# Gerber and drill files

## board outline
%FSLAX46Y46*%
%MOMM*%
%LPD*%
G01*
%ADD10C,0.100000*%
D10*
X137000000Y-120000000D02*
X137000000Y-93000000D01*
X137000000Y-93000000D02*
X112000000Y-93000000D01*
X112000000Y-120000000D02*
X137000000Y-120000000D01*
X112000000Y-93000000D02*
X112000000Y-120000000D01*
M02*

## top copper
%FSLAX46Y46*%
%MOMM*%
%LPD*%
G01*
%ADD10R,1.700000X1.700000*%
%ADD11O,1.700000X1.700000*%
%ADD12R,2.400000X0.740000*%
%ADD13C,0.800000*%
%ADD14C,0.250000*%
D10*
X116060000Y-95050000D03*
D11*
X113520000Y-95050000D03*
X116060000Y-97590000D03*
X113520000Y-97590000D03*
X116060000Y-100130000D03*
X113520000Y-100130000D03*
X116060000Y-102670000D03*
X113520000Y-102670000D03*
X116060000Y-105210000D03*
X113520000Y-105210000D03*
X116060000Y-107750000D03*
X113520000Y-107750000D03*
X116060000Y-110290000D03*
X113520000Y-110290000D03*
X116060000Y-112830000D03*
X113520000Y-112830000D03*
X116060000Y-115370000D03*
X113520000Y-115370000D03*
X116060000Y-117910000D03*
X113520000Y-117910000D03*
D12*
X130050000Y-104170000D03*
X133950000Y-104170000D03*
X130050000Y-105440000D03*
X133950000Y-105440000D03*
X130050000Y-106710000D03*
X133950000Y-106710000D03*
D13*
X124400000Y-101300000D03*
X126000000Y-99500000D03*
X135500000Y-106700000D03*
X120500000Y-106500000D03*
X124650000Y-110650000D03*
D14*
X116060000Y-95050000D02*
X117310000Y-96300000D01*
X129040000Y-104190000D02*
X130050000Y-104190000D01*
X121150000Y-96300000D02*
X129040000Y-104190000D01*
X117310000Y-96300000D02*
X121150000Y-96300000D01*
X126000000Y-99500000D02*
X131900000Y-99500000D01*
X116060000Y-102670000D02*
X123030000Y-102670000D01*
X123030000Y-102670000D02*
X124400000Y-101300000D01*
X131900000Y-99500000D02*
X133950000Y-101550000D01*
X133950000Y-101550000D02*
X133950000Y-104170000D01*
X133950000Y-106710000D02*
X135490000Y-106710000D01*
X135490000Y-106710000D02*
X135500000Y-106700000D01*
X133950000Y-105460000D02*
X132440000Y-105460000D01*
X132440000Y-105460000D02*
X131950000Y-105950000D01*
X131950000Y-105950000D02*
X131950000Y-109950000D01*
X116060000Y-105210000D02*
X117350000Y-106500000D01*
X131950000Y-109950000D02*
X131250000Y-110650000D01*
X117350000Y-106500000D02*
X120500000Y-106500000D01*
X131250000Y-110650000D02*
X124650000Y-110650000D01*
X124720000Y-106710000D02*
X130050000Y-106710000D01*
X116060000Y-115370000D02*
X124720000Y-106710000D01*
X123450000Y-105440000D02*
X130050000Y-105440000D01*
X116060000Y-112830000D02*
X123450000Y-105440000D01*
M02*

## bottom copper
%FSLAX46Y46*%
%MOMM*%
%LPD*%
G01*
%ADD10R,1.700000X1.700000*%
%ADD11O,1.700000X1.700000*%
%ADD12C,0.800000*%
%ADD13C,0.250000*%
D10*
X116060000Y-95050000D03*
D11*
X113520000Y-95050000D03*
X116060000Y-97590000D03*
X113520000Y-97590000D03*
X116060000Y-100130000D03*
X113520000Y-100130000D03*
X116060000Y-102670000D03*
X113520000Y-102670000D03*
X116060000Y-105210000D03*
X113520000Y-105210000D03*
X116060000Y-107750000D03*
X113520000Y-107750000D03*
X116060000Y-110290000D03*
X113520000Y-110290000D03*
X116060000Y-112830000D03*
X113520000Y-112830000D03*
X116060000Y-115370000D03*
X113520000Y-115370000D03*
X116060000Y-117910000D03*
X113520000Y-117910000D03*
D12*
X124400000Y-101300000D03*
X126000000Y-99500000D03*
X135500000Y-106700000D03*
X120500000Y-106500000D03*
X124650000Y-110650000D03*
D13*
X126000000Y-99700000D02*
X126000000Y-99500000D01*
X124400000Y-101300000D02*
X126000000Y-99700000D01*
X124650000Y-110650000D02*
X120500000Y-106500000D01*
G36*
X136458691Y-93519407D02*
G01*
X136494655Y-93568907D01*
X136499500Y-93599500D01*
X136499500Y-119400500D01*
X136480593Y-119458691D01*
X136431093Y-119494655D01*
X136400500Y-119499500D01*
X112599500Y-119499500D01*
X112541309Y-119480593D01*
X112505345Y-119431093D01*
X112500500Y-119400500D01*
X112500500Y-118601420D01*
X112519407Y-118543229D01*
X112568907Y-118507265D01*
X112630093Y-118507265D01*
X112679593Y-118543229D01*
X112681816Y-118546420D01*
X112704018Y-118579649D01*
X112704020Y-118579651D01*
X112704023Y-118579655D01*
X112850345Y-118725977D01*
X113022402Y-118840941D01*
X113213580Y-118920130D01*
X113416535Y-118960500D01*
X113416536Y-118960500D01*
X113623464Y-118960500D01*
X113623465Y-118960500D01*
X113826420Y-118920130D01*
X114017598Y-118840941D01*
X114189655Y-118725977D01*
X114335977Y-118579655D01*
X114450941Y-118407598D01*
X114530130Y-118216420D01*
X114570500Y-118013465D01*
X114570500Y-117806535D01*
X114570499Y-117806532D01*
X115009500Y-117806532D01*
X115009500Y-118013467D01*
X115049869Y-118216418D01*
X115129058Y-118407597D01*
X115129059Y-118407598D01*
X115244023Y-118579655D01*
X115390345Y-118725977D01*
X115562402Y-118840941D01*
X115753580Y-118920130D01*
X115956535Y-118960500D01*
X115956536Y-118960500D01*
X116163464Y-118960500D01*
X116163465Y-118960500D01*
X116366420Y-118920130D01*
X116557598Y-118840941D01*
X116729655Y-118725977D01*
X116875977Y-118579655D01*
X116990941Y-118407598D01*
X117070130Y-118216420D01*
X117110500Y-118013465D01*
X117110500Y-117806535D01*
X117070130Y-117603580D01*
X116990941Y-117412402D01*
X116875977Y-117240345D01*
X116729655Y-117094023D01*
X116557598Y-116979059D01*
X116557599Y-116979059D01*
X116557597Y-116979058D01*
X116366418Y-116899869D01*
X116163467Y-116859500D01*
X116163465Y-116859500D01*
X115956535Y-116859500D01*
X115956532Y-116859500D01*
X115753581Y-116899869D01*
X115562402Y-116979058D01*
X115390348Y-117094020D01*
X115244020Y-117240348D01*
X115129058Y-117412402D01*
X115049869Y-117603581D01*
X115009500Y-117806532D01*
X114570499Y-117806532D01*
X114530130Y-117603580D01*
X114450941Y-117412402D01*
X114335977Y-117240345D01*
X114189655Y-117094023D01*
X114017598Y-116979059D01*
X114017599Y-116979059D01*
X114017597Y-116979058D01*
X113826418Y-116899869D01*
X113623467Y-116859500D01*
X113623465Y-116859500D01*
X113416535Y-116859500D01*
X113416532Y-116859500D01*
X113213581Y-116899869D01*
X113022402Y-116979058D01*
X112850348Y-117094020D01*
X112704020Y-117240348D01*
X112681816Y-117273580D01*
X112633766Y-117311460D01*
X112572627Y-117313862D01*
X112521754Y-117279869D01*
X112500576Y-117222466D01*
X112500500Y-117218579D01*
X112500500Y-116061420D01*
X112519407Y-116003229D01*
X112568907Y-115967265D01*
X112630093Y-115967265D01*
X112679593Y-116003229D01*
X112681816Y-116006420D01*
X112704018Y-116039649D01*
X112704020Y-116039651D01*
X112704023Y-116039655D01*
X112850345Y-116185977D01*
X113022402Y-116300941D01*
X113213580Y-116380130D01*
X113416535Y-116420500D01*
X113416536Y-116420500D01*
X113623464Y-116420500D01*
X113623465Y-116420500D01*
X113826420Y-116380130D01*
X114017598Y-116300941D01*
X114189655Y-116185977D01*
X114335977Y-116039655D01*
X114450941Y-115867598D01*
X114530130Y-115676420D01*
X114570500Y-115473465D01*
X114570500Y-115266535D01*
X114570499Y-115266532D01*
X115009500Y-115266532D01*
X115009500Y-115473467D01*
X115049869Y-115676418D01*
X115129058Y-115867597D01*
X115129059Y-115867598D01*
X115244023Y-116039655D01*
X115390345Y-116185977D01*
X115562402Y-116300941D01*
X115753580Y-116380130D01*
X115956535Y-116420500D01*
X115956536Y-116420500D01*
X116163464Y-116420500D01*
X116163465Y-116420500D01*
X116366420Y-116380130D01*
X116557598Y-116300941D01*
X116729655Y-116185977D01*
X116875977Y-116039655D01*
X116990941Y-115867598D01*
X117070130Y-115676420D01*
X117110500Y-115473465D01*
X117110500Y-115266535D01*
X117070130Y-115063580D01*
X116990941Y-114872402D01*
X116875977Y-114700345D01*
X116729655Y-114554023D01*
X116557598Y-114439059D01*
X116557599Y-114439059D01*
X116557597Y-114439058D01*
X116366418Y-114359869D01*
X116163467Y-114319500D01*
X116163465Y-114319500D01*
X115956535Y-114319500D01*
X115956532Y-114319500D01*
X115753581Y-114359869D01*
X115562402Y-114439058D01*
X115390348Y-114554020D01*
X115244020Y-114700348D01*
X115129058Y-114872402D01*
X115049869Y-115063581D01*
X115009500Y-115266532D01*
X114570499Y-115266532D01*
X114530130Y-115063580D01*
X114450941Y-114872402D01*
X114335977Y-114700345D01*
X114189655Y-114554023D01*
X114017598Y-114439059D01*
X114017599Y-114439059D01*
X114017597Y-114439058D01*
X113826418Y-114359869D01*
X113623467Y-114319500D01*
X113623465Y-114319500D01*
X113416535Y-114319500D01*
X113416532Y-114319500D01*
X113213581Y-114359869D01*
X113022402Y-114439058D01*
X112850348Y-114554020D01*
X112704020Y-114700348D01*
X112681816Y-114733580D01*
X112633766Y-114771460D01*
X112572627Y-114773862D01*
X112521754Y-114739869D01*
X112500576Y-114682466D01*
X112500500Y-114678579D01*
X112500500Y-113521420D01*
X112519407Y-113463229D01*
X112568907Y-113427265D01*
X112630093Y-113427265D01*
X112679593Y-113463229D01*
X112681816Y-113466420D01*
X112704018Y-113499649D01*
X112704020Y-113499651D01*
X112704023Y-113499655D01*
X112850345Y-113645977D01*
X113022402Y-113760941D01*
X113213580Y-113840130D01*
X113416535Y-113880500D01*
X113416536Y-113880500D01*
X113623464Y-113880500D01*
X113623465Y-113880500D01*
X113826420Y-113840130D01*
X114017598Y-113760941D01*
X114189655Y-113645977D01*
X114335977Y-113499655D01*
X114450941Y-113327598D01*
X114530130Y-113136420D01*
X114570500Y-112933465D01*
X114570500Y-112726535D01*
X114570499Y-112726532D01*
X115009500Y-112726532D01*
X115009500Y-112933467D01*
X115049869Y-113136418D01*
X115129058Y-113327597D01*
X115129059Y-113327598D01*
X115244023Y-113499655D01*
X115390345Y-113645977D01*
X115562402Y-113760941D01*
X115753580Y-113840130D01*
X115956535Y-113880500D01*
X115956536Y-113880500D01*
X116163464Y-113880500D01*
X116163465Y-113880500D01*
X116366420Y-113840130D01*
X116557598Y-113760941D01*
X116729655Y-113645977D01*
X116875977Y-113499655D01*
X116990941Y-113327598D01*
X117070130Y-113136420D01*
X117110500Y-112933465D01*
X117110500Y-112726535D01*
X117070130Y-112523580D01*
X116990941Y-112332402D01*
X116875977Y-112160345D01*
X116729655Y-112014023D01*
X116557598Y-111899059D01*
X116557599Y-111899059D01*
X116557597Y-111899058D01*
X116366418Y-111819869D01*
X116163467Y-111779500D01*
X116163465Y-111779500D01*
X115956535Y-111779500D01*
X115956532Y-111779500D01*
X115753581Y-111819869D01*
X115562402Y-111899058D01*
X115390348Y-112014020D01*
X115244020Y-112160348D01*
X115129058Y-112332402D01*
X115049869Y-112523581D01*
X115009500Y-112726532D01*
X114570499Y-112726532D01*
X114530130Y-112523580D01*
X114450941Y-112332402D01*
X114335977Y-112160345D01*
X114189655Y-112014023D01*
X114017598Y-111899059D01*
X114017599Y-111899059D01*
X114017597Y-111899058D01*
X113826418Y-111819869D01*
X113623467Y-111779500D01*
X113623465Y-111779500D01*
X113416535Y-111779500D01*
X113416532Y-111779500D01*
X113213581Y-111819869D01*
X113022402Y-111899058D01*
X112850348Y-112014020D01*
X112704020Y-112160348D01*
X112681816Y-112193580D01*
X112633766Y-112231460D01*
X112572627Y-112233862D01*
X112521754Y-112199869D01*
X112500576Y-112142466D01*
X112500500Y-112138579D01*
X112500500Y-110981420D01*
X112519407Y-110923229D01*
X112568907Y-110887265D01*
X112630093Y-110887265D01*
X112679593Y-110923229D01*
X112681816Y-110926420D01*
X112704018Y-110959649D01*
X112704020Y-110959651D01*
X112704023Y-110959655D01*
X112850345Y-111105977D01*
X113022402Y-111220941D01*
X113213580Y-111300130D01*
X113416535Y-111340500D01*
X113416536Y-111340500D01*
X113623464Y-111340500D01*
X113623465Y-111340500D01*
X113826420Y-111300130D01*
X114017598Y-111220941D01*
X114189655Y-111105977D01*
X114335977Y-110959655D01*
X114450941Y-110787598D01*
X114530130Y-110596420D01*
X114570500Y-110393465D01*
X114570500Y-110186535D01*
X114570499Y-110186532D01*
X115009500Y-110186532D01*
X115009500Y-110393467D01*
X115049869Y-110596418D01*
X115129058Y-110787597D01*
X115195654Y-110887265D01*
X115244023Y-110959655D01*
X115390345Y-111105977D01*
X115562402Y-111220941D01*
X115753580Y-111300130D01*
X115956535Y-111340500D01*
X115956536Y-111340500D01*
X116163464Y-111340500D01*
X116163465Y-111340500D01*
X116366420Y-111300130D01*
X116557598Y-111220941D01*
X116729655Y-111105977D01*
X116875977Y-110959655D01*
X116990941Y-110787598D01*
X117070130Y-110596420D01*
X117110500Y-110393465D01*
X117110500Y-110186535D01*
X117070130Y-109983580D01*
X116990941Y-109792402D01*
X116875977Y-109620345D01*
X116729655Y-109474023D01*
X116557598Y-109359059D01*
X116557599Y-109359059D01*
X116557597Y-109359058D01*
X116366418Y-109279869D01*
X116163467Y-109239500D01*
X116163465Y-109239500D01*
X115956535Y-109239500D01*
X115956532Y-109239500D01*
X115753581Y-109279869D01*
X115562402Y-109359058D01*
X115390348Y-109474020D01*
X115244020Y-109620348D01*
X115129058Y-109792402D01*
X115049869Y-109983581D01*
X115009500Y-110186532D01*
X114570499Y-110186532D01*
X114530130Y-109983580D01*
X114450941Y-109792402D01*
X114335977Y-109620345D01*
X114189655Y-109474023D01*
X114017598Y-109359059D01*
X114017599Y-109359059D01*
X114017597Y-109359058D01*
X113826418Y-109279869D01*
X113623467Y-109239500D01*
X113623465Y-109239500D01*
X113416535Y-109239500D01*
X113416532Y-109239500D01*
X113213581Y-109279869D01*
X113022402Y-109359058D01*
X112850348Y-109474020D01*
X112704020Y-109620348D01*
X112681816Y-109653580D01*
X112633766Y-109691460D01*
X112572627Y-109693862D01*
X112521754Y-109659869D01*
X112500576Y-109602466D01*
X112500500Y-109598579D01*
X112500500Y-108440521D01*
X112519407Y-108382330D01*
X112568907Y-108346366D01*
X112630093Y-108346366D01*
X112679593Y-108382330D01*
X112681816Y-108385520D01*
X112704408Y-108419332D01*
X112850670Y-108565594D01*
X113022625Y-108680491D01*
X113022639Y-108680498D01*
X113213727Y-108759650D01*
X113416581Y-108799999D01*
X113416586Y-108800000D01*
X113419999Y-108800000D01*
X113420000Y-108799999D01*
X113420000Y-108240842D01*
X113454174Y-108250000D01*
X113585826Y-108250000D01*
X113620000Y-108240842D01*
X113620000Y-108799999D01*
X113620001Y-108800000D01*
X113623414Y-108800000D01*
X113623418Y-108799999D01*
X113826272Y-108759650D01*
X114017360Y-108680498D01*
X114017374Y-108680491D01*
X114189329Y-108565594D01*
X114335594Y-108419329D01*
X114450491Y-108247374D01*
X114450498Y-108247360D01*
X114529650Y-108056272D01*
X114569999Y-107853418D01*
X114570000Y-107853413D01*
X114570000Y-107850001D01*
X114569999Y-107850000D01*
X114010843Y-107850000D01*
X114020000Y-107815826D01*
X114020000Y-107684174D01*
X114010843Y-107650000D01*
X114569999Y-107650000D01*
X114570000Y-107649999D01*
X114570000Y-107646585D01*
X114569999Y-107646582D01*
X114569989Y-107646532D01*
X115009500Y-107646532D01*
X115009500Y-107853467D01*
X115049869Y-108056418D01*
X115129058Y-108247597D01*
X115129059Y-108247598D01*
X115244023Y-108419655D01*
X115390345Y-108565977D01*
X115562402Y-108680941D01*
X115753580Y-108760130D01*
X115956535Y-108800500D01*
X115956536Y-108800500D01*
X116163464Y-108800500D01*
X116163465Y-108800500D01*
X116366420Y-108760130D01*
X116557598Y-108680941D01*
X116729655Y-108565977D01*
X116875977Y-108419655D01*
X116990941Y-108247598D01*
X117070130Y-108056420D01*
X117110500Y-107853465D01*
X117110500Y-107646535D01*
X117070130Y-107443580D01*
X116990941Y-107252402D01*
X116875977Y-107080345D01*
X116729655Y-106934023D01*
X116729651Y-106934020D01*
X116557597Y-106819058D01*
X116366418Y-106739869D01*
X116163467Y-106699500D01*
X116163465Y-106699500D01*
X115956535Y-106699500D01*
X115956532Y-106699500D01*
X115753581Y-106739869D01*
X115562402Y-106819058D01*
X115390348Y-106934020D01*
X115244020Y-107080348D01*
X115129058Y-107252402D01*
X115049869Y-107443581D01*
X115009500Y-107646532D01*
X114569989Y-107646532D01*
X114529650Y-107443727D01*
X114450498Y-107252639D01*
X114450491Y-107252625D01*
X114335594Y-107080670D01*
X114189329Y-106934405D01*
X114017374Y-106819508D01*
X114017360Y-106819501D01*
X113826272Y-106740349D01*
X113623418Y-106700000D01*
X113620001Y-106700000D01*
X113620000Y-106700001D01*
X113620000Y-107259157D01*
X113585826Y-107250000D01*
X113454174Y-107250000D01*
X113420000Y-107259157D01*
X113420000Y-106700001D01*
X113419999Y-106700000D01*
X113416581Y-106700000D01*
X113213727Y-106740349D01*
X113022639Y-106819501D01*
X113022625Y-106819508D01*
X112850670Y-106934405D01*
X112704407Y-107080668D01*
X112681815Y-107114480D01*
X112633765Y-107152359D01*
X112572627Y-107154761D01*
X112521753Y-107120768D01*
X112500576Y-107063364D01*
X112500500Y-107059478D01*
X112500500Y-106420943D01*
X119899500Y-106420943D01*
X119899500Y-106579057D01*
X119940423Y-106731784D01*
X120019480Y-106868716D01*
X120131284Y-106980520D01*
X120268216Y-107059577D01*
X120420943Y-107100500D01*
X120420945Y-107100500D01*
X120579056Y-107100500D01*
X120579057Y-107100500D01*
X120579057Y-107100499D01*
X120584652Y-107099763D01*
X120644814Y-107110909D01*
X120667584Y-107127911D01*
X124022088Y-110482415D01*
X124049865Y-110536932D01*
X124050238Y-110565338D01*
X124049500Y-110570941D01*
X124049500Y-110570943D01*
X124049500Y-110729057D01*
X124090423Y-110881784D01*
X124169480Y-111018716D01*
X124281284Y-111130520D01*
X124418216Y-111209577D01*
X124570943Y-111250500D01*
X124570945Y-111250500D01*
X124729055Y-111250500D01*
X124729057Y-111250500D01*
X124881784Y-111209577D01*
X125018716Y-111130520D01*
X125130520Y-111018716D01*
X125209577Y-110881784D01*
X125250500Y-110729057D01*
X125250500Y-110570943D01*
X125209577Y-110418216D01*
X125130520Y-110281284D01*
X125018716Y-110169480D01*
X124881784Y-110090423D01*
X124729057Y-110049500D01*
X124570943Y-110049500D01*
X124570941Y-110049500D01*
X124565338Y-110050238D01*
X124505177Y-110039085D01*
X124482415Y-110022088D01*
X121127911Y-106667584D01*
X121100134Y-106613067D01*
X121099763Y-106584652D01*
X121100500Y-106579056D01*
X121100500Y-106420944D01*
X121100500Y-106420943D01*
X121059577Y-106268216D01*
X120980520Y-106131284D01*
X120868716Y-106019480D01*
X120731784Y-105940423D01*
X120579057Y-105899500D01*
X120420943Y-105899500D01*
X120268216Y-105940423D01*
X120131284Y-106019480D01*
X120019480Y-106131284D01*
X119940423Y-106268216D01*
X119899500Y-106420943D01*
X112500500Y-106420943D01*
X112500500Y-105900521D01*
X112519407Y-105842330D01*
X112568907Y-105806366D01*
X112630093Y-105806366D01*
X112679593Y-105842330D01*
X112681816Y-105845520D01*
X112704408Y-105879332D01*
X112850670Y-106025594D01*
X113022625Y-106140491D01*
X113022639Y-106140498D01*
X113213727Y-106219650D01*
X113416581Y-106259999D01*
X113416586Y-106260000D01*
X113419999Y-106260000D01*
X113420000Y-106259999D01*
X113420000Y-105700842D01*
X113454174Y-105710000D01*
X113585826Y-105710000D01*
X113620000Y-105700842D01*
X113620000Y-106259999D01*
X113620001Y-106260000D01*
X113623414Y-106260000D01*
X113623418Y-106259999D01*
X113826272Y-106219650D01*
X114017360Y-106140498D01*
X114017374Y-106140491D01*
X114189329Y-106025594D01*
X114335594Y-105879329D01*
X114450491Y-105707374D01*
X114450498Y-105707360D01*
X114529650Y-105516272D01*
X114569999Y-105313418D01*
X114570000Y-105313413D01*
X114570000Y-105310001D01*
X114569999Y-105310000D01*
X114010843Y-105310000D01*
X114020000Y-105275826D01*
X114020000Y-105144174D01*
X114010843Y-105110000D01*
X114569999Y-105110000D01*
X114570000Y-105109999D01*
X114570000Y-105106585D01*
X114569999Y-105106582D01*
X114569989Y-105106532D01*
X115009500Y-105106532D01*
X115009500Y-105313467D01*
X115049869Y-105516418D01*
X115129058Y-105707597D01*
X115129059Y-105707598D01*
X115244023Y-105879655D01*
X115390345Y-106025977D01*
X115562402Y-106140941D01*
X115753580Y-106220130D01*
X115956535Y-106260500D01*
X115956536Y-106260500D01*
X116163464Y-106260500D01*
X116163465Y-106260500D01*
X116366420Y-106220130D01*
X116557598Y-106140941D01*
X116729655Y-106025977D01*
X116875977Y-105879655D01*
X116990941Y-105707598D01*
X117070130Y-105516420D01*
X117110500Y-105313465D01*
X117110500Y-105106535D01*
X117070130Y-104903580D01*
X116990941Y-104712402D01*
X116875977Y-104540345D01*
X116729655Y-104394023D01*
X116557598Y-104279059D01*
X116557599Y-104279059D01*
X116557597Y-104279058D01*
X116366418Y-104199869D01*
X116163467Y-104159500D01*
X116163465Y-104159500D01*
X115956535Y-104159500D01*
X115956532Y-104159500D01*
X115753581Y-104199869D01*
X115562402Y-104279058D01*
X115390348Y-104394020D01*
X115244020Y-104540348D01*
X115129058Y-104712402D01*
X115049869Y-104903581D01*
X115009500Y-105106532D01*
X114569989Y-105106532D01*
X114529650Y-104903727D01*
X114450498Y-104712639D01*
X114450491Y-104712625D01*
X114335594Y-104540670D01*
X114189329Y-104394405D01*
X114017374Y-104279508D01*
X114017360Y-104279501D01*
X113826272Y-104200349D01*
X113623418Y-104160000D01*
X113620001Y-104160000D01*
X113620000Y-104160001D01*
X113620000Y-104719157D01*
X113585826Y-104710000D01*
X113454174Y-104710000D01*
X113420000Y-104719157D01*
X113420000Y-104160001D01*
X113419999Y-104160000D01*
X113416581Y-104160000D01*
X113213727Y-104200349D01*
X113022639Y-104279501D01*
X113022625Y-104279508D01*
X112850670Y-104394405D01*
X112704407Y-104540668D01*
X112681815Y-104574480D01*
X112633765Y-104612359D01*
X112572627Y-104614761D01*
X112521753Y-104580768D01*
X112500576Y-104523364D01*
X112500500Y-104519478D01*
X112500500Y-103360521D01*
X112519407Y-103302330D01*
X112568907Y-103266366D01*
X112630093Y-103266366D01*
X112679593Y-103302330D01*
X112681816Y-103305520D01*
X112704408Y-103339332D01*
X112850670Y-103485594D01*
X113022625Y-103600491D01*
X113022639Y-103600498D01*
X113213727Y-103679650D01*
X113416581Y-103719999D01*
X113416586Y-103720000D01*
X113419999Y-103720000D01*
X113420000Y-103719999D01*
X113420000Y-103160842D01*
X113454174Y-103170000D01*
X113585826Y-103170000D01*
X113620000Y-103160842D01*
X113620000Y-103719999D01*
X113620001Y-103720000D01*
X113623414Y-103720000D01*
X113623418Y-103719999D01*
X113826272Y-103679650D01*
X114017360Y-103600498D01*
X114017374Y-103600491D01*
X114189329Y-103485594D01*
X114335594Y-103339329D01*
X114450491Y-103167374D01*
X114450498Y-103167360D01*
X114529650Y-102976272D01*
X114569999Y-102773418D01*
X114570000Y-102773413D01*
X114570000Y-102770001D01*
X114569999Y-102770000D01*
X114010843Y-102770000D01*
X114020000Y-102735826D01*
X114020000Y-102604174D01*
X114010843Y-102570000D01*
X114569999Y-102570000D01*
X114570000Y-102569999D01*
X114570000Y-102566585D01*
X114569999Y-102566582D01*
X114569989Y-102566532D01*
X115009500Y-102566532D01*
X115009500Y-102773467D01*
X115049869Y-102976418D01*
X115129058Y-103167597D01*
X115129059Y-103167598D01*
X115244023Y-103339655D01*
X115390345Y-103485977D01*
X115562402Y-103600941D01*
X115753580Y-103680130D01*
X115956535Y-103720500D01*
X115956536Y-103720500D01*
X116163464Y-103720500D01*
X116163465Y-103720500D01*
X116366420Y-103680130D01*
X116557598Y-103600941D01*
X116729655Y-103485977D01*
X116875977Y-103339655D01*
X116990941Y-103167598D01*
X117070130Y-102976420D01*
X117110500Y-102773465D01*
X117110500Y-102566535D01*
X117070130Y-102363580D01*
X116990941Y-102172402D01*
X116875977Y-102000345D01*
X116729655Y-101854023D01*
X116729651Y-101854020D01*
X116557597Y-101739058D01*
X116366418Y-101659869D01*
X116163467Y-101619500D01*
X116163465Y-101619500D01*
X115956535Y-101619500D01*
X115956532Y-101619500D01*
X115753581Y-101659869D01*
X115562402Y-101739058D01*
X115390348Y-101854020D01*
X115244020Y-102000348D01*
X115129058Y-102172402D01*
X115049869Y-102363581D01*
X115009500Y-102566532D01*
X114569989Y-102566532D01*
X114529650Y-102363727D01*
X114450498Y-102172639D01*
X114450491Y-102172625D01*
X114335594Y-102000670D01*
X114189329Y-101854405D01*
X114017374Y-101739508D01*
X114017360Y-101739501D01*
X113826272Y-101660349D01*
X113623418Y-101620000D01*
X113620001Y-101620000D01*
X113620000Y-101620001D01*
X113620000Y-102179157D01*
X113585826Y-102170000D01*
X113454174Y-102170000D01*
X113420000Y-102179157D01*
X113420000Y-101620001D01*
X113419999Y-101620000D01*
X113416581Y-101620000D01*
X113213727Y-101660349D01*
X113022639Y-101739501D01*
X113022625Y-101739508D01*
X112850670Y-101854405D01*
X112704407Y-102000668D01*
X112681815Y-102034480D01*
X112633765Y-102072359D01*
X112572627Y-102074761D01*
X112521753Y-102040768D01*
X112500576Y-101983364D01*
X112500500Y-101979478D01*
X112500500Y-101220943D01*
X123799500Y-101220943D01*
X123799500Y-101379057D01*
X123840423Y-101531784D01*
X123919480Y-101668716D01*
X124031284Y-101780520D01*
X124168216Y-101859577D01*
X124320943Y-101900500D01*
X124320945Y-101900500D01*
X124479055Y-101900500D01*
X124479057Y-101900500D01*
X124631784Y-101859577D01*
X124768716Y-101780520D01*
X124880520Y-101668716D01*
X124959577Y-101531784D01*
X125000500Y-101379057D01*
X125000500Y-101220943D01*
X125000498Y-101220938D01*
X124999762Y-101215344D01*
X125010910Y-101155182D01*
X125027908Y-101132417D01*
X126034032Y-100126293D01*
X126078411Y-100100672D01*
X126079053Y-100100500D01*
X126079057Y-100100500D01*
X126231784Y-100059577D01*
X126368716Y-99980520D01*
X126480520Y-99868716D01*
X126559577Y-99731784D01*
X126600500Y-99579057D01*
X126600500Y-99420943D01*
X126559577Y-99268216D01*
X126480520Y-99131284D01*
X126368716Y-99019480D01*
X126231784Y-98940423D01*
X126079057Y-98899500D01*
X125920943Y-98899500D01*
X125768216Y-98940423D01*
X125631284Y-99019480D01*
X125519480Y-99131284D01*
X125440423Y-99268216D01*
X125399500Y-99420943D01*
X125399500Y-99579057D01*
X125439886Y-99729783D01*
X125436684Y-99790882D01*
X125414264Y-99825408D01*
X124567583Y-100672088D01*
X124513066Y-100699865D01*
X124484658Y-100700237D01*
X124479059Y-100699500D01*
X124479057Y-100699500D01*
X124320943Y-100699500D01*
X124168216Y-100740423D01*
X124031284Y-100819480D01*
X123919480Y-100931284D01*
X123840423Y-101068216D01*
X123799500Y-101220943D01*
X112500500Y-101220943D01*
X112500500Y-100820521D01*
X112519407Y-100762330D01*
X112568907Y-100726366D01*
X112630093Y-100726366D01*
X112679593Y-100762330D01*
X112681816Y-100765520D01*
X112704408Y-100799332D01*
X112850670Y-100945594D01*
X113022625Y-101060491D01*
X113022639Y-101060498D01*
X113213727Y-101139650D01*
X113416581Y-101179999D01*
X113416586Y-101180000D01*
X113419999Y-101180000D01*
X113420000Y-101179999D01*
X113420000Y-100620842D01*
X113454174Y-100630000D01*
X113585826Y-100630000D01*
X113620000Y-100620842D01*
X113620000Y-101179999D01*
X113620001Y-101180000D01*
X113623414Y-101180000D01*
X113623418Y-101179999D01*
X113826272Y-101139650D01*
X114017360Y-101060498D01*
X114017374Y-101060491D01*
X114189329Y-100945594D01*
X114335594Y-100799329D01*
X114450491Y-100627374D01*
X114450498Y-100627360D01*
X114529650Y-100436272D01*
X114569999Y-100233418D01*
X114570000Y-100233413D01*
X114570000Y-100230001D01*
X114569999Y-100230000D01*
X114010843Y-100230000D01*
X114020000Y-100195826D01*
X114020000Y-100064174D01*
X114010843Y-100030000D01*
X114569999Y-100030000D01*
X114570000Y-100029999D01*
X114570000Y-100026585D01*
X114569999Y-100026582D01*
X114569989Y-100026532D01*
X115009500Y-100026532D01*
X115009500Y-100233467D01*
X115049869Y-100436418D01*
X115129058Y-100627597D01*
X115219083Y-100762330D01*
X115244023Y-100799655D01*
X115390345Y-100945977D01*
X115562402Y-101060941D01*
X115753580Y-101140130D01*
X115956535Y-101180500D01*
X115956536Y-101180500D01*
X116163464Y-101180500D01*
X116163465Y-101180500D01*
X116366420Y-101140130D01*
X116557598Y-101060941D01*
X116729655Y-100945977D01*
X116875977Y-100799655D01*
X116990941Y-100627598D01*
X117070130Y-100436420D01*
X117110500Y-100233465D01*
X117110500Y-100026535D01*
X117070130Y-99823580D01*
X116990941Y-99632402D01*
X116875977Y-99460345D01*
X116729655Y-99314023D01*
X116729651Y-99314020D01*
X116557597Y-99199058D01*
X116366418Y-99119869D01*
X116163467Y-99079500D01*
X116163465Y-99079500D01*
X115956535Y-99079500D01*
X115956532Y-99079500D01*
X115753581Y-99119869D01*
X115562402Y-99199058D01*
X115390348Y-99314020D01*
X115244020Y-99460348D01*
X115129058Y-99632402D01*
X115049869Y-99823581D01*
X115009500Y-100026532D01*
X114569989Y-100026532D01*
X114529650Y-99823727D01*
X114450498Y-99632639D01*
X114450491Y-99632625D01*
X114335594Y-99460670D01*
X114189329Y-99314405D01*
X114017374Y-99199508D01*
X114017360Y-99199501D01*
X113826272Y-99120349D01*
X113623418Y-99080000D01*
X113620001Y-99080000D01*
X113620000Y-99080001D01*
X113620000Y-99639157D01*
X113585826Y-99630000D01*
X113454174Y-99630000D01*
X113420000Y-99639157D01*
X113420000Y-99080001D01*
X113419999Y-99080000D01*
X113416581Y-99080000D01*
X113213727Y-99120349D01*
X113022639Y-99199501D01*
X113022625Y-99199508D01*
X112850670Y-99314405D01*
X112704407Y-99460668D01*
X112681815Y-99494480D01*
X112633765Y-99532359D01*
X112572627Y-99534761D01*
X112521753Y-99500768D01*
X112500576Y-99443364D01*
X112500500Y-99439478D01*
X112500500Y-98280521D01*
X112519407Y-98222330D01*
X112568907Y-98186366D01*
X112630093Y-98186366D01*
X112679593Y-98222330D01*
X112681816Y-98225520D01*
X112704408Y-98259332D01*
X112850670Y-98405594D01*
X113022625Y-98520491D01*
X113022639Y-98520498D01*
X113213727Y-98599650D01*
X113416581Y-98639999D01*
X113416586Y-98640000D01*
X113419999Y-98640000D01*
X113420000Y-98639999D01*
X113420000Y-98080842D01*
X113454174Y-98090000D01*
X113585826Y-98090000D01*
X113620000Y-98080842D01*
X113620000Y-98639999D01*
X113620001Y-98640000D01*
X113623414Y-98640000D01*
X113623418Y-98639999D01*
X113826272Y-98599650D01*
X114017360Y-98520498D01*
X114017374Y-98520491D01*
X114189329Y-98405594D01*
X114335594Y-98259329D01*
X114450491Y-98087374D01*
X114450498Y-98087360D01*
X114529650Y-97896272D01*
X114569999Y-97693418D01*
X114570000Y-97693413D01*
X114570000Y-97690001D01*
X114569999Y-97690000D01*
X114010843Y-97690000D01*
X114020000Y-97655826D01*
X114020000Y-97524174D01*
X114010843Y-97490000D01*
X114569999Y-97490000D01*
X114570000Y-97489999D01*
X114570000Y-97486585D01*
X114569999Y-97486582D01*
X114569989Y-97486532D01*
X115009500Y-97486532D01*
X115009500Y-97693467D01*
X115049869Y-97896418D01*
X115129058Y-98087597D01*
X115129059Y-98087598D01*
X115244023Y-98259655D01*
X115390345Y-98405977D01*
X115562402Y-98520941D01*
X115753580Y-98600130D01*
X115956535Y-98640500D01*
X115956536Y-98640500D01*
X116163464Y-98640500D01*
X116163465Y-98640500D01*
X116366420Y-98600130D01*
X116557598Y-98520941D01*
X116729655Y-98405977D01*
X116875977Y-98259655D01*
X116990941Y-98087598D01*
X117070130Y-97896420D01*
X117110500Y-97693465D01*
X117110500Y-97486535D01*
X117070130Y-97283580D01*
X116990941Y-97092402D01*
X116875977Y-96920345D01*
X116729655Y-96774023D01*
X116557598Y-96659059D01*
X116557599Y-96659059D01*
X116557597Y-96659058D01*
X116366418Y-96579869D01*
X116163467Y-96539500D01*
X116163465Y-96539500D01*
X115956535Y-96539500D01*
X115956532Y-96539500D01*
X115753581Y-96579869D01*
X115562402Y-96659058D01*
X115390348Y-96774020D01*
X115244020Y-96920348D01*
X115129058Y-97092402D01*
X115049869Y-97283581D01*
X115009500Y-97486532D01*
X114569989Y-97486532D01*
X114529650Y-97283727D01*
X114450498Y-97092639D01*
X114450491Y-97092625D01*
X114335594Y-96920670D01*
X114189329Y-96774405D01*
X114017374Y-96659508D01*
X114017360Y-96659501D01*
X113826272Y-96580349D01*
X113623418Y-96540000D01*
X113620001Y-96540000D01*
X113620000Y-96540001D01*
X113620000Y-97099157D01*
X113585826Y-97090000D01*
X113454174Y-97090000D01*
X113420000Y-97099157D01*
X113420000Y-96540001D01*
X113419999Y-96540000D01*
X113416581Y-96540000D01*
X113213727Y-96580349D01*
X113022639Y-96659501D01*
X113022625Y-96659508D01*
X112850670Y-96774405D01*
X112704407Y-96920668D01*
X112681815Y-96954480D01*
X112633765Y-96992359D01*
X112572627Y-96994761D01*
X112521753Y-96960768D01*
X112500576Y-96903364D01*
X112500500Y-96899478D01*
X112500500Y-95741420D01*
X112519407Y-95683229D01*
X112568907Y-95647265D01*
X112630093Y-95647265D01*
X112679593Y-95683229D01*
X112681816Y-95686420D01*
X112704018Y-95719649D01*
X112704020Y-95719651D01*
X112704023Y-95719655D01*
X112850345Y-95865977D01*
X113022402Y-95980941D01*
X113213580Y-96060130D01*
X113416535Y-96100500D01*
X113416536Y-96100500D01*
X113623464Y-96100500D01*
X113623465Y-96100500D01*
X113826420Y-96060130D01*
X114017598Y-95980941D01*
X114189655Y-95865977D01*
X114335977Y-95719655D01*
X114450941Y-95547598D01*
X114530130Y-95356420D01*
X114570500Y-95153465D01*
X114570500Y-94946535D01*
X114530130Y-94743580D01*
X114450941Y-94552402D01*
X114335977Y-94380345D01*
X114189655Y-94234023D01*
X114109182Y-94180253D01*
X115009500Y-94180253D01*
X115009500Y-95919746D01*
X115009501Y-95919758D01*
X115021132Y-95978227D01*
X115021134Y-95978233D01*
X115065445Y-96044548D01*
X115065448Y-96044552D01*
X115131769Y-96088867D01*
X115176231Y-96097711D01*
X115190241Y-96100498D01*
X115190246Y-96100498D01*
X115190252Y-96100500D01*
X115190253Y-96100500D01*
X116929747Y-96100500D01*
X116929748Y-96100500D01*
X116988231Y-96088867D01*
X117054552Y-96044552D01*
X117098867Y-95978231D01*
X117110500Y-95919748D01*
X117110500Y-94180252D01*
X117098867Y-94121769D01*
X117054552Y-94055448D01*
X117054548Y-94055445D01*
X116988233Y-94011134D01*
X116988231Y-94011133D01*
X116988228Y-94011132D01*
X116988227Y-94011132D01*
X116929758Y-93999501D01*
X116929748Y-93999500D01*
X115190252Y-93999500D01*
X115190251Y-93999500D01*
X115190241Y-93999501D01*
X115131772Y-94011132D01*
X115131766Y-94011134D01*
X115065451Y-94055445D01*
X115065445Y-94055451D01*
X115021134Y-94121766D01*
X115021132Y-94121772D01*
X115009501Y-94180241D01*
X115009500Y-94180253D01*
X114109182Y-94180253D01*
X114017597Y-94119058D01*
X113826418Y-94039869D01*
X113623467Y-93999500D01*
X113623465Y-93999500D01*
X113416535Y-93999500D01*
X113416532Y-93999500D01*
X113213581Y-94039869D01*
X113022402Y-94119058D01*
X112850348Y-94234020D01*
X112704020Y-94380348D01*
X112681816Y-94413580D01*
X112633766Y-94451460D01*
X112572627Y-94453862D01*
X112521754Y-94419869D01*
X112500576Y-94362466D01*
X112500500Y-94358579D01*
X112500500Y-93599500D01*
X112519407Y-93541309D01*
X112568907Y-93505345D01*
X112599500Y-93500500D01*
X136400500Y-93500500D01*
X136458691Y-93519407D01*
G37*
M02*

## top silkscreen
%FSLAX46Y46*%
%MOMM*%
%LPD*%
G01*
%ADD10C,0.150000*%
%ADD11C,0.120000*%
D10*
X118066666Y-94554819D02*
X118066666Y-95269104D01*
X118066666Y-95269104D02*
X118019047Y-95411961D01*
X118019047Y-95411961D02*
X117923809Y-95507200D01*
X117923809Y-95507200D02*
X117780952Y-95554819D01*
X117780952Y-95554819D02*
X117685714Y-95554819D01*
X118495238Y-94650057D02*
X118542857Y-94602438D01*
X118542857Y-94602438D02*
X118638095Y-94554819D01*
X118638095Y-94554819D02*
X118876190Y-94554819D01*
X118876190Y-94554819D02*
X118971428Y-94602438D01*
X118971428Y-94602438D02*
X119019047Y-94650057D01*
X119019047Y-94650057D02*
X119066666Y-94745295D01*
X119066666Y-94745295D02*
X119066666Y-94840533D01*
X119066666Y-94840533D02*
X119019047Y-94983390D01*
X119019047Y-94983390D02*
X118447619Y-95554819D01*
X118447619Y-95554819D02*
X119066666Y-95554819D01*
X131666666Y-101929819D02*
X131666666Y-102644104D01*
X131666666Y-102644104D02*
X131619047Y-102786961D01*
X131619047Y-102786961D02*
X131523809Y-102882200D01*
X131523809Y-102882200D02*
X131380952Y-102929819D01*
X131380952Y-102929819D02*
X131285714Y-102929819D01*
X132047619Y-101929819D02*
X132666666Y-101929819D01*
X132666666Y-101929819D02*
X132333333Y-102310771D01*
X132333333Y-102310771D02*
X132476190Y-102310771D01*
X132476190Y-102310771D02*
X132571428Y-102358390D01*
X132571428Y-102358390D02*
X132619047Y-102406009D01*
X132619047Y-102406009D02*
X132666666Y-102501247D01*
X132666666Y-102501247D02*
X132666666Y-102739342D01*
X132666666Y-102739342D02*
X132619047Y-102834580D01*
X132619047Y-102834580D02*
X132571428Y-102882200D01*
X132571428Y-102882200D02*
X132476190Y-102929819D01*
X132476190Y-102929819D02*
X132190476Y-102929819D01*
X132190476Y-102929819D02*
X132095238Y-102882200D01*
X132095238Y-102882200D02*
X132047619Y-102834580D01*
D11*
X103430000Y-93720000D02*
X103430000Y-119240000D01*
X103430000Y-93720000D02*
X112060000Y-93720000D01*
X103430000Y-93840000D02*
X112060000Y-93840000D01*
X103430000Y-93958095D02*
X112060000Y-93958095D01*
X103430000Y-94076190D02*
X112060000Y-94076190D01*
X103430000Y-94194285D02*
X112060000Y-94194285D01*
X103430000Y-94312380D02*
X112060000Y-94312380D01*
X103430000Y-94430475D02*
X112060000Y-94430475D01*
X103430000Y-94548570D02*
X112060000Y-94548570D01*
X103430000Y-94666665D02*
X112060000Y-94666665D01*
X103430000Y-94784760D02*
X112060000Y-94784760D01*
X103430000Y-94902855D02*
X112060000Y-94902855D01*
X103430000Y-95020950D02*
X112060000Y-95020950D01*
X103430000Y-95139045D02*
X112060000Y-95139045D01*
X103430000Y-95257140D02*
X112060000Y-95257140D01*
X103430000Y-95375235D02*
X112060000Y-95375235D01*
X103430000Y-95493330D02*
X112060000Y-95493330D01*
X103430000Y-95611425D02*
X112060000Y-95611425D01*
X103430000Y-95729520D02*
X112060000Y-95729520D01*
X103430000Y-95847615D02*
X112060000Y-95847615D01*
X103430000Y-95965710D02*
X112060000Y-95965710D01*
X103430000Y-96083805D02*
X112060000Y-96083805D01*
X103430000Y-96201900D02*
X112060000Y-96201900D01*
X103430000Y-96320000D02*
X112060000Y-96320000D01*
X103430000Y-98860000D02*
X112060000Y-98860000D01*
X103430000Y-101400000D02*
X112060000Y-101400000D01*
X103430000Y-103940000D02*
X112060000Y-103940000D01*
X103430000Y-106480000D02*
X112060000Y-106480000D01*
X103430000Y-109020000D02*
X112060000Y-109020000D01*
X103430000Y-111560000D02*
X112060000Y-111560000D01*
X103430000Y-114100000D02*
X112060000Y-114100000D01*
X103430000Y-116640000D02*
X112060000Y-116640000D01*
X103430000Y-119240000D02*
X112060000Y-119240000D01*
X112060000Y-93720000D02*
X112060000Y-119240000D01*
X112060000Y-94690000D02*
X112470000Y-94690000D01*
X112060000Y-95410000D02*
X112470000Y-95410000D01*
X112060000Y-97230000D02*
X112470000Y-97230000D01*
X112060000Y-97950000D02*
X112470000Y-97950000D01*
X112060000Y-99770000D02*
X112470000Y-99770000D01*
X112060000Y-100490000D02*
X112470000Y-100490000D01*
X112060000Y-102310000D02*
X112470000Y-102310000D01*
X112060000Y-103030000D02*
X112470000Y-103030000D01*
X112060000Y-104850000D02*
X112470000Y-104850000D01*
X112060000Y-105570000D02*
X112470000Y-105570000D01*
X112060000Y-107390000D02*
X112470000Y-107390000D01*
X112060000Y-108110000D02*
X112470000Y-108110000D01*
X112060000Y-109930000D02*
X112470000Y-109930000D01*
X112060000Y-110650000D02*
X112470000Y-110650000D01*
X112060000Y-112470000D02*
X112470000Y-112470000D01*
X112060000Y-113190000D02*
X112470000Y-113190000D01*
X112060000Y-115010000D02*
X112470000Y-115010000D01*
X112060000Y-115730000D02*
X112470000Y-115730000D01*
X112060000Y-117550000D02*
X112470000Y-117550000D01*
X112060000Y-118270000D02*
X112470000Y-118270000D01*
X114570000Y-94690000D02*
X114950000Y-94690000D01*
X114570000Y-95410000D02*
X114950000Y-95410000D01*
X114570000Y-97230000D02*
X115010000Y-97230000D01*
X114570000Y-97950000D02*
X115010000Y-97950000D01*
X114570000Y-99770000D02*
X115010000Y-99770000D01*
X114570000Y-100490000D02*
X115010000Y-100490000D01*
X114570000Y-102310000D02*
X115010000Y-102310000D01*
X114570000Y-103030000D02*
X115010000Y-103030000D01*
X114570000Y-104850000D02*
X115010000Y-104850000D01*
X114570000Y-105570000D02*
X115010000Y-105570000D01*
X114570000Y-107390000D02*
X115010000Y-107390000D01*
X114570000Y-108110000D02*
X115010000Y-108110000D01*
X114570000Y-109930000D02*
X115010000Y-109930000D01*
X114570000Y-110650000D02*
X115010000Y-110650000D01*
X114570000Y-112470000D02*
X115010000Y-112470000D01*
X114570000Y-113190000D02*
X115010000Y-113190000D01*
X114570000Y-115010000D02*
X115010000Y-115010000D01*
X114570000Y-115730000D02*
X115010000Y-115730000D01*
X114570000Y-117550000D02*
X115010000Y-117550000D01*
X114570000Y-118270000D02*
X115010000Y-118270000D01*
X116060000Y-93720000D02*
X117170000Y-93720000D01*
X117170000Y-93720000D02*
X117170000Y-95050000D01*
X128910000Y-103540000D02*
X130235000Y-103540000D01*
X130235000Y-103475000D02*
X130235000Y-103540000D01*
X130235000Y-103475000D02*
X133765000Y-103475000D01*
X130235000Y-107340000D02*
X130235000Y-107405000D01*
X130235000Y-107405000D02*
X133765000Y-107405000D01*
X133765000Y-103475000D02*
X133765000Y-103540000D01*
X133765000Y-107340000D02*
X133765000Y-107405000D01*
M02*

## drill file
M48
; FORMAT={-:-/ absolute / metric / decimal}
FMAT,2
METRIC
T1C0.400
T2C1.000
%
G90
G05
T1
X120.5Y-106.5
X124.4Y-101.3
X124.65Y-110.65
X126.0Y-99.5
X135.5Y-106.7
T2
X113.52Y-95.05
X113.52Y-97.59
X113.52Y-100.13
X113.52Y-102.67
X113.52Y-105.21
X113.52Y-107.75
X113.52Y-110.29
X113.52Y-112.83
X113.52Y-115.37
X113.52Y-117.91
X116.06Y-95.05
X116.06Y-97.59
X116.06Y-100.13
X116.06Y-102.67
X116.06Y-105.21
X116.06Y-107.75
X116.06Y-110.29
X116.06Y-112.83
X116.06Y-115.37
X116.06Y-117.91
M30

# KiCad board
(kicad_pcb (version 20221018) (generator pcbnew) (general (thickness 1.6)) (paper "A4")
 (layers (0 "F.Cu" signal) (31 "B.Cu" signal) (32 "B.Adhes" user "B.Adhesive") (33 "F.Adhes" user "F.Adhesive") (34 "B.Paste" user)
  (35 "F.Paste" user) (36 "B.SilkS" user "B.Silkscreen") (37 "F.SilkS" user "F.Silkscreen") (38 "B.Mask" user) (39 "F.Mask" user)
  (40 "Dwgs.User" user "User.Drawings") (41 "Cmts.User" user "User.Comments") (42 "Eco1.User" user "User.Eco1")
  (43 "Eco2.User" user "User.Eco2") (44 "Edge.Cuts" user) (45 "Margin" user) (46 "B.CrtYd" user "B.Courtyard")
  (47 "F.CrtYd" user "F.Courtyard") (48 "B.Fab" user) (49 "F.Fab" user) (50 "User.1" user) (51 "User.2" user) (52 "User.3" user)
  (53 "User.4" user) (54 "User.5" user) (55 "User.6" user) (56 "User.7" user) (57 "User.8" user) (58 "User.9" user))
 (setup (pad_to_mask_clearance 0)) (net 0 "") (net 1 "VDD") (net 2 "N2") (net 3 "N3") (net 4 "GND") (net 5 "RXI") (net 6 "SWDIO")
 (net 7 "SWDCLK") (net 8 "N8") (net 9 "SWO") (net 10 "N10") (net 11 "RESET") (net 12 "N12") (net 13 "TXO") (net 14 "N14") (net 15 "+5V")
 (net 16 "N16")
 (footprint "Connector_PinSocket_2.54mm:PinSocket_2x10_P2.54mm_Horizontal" (layer "F.Cu") (at 116.06 95.05)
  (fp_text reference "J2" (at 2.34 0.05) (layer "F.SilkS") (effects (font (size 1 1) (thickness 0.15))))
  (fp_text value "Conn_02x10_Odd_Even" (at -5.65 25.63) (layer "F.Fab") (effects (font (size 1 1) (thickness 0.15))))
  (fp_line (start -12.63 -1.33) (end -12.63 24.19) (stroke (width 0.12) (type solid)) (layer "F.SilkS"))
  (fp_line (start -12.63 -1.33) (end -4 -1.33) (stroke (width 0.12) (type solid)) (layer "F.SilkS"))
  (fp_line (start -12.63 -1.21) (end -4 -1.21) (stroke (width 0.12) (type solid)) (layer "F.SilkS"))
  (fp_line (start -12.63 -1.091905) (end -4 -1.091905) (stroke (width 0.12) (type solid)) (layer "F.SilkS"))
  (fp_line (start -12.63 -0.97381) (end -4 -0.97381) (stroke (width 0.12) (type solid)) (layer "F.SilkS"))
  (fp_line (start -12.63 -0.855715) (end -4 -0.855715) (stroke (width 0.12) (type solid)) (layer "F.SilkS"))
  (fp_line (start -12.63 -0.73762) (end -4 -0.73762) (stroke (width 0.12) (type solid)) (layer "F.SilkS"))
  (fp_line (start -12.63 -0.619525) (end -4 -0.619525) (stroke (width 0.12) (type solid)) (layer "F.SilkS"))
  (fp_line (start -12.63 -0.50143) (end -4 -0.50143) (stroke (width 0.12) (type solid)) (layer "F.SilkS"))
  (fp_line (start -12.63 -0.383335) (end -4 -0.383335) (stroke (width 0.12) (type solid)) (layer "F.SilkS"))
  (fp_line (start -12.63 -0.26524) (end -4 -0.26524) (stroke (width 0.12) (type solid)) (layer "F.SilkS"))
  (fp_line (start -12.63 -0.147145) (end -4 -0.147145) (stroke (width 0.12) (type solid)) (layer "F.SilkS"))
  (fp_line (start -12.63 -0.02905) (end -4 -0.02905) (stroke (width 0.12) (type solid)) (layer "F.SilkS"))
  (fp_line (start -12.63 0.089045) (end -4 0.089045) (stroke (width 0.12) (type solid)) (layer "F.SilkS"))
  (fp_line (start -12.63 0.20714) (end -4 0.20714) (stroke (width 0.12) (type solid)) (layer "F.SilkS"))
  (fp_line (start -12.63 0.325235) (end -4 0.325235) (stroke (width 0.12) (type solid)) (layer "F.SilkS"))
  (fp_line (start -12.63 0.44333) (end -4 0.44333) (stroke (width 0.12) (type solid)) (layer "F.SilkS"))
  (fp_line (start -12.63 0.561425) (end -4 0.561425) (stroke (width 0.12) (type solid)) (layer "F.SilkS"))
  (fp_line (start -12.63 0.67952) (end -4 0.67952) (stroke (width 0.12) (type solid)) (layer "F.SilkS"))
  (fp_line (start -12.63 0.797615) (end -4 0.797615) (stroke (width 0.12) (type solid)) (layer "F.SilkS"))
  (fp_line (start -12.63 0.91571) (end -4 0.91571) (stroke (width 0.12) (type solid)) (layer "F.SilkS"))
  (fp_line (start -12.63 1.033805) (end -4 1.033805) (stroke (width 0.12) (type solid)) (layer "F.SilkS"))
  (fp_line (start -12.63 1.1519) (end -4 1.1519) (stroke (width 0.12) (type solid)) (layer "F.SilkS"))
  (fp_line (start -12.63 1.27) (end -4 1.27) (stroke (width 0.12) (type solid)) (layer "F.SilkS"))
  (fp_line (start -12.63 3.81) (end -4 3.81) (stroke (width 0.12) (type solid)) (layer "F.SilkS"))
  (fp_line (start -12.63 6.35) (end -4 6.35) (stroke (width 0.12) (type solid)) (layer "F.SilkS"))
  (fp_line (start -12.63 8.89) (end -4 8.89) (stroke (width 0.12) (type solid)) (layer "F.SilkS"))
  (fp_line (start -12.63 11.43) (end -4 11.43) (stroke (width 0.12) (type solid)) (layer "F.SilkS"))
  (fp_line (start -12.63 13.97) (end -4 13.97) (stroke (width 0.12) (type solid)) (layer "F.SilkS"))
  (fp_line (start -12.63 16.51) (end -4 16.51) (stroke (width 0.12) (type solid)) (layer "F.SilkS"))
  (fp_line (start -12.63 19.05) (end -4 19.05) (stroke (width 0.12) (type solid)) (layer "F.SilkS"))
  (fp_line (start -12.63 21.59) (end -4 21.59) (stroke (width 0.12) (type solid)) (layer "F.SilkS"))
  (fp_line (start -12.63 24.19) (end -4 24.19) (stroke (width 0.12) (type solid)) (layer "F.SilkS"))
  (fp_line (start -4 -1.33) (end -4 24.19) (stroke (width 0.12) (type solid)) (layer "F.SilkS"))
  (fp_line (start -4 -0.36) (end -3.59 -0.36) (stroke (width 0.12) (type solid)) (layer "F.SilkS"))
  (fp_line (start -4 0.36) (end -3.59 0.36) (stroke (width 0.12) (type solid)) (layer "F.SilkS"))
  (fp_line (start -4 2.18) (end -3.59 2.18) (stroke (width 0.12) (type solid)) (layer "F.SilkS"))
  (fp_line (start -4 2.9) (end -3.59 2.9) (stroke (width 0.12) (type solid)) (layer "F.SilkS"))
  (fp_line (start -4 4.72) (end -3.59 4.72) (stroke (width 0.12) (type solid)) (layer "F.SilkS"))
  (fp_line (start -4 5.44) (end -3.59 5.44) (stroke (width 0.12) (type solid)) (layer "F.SilkS"))
  (fp_line (start -4 7.26) (end -3.59 7.26) (stroke (width 0.12) (type solid)) (layer "F.SilkS"))
  (fp_line (start -4 7.98) (end -3.59 7.98) (stroke (width 0.12) (type solid)) (layer "F.SilkS"))
  (fp_line (start -4 9.8) (end -3.59 9.8) (stroke (width 0.12) (type solid)) (layer "F.SilkS"))
  (fp_line (start -4 10.52) (end -3.59 10.52) (stroke (width 0.12) (type solid)) (layer "F.SilkS"))
  (fp_line (start -4 12.34) (end -3.59 12.34) (stroke (width 0.12) (type solid)) (layer "F.SilkS"))
  (fp_line (start -4 13.06) (end -3.59 13.06) (stroke (width 0.12) (type solid)) (layer "F.SilkS"))
  (fp_line (start -4 14.88) (end -3.59 14.88) (stroke (width 0.12) (type solid)) (layer "F.SilkS"))
  (fp_line (start -4 15.6) (end -3.59 15.6) (stroke (width 0.12) (type solid)) (layer "F.SilkS"))
  (fp_line (start -4 17.42) (end -3.59 17.42) (stroke (width 0.12) (type solid)) (layer "F.SilkS"))
  (fp_line (start -4 18.14) (end -3.59 18.14) (stroke (width 0.12) (type solid)) (layer "F.SilkS"))
  (fp_line (start -4 19.96) (end -3.59 19.96) (stroke (width 0.12) (type solid)) (layer "F.SilkS"))
  (fp_line (start -4 20.68) (end -3.59 20.68) (stroke (width 0.12) (type solid)) (layer "F.SilkS"))
  (fp_line (start -4 22.5) (end -3.59 22.5) (stroke (width 0.12) (type solid)) (layer "F.SilkS"))
  (fp_line (start -4 23.22) (end -3.59 23.22) (stroke (width 0.12) (type solid)) (layer "F.SilkS"))
  (fp_line (start -1.49 -0.36) (end -1.11 -0.36) (stroke (width 0.12) (type solid)) (layer "F.SilkS"))
  (fp_line (start -1.49 0.36) (end -1.11 0.36) (stroke (width 0.12) (type solid)) (layer "F.SilkS"))
  (fp_line (start -1.49 2.18) (end -1.05 2.18) (stroke (width 0.12) (type solid)) (layer "F.SilkS"))
  (fp_line (start -1.49 2.9) (end -1.05 2.9) (stroke (width 0.12) (type solid)) (layer "F.SilkS"))
  (fp_line (start -1.49 4.72) (end -1.05 4.72) (stroke (width 0.12) (type solid)) (layer "F.SilkS"))
  (fp_line (start -1.49 5.44) (end -1.05 5.44) (stroke (width 0.12) (type solid)) (layer "F.SilkS"))
  (fp_line (start -1.49 7.26) (end -1.05 7.26) (stroke (width 0.12) (type solid)) (layer "F.SilkS"))
  (fp_line (start -1.49 7.98) (end -1.05 7.98) (stroke (width 0.12) (type solid)) (layer "F.SilkS"))
  (fp_line (start -1.49 9.8) (end -1.05 9.8) (stroke (width 0.12) (type solid)) (layer "F.SilkS"))
  (fp_line (start -1.49 10.52) (end -1.05 10.52) (stroke (width 0.12) (type solid)) (layer "F.SilkS"))
  (fp_line (start -1.49 12.34) (end -1.05 12.34) (stroke (width 0.12) (type solid)) (layer "F.SilkS"))
  (fp_line (start -1.49 13.06) (end -1.05 13.06) (stroke (width 0.12) (type solid)) (layer "F.SilkS"))
  (fp_line (start -1.49 14.88) (end -1.05 14.88) (stroke (width 0.12) (type solid)) (layer "F.SilkS"))
  (fp_line (start -1.49 15.6) (end -1.05 15.6) (stroke (width 0.12) (type solid)) (layer "F.SilkS"))
  (fp_line (start -1.49 17.42) (end -1.05 17.42) (stroke (width 0.12) (type solid)) (layer "F.SilkS"))
  (fp_line (start -1.49 18.14) (end -1.05 18.14) (stroke (width 0.12) (type solid)) (layer "F.SilkS"))
  (fp_line (start -1.49 19.96) (end -1.05 19.96) (stroke (width 0.12) (type solid)) (layer "F.SilkS"))
  (fp_line (start -1.49 20.68) (end -1.05 20.68) (stroke (width 0.12) (type solid)) (layer "F.SilkS"))
  (fp_line (start -1.49 22.5) (end -1.05 22.5) (stroke (width 0.12) (type solid)) (layer "F.SilkS"))
  (fp_line (start -1.49 23.22) (end -1.05 23.22) (stroke (width 0.12) (type solid)) (layer "F.SilkS"))
  (fp_line (start 0 -1.33) (end 1.11 -1.33) (stroke (width 0.12) (type solid)) (layer "F.SilkS"))
  (fp_line (start 1.11 -1.33) (end 1.11 0) (stroke (width 0.12) (type solid)) (layer "F.SilkS"))
  (pad "1" thru_hole rect (at 0 0) (size 1.7 1.7) (drill 1) (layers "*.Cu" "*.Mask") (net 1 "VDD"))
  (pad "2" thru_hole oval (at -2.54 0) (size 1.7 1.7) (drill 1) (layers "*.Cu" "*.Mask") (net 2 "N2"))
  (pad "3" thru_hole oval (at 0 2.54) (size 1.7 1.7) (drill 1) (layers "*.Cu" "*.Mask") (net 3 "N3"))
  (pad "4" thru_hole oval (at -2.54 2.54) (size 1.7 1.7) (drill 1) (layers "*.Cu" "*.Mask") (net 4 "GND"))
  (pad "5" thru_hole oval (at 0 5.08) (size 1.7 1.7) (drill 1) (layers "*.Cu" "*.Mask") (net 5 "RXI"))
  (pad "6" thru_hole oval (at -2.54 5.08) (size 1.7 1.7) (drill 1) (layers "*.Cu" "*.Mask") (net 4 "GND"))
  (pad "7" thru_hole oval (at 0 7.62) (size 1.7 1.7) (drill 1) (layers "*.Cu" "*.Mask") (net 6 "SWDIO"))
  (pad "8" thru_hole oval (at -2.54 7.62) (size 1.7 1.7) (drill 1) (layers "*.Cu" "*.Mask") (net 4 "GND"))
  (pad "9" thru_hole oval (at 0 10.16) (size 1.7 1.7) (drill 1) (layers "*.Cu" "*.Mask") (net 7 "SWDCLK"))
  (pad "10" thru_hole oval (at -2.54 10.16) (size 1.7 1.7) (drill 1) (layers "*.Cu" "*.Mask") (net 4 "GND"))
  (pad "11" thru_hole oval (at 0 12.7) (size 1.7 1.7) (drill 1) (layers "*.Cu" "*.Mask") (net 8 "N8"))
  (pad "12" thru_hole oval (at -2.54 12.7) (size 1.7 1.7) (drill 1) (layers "*.Cu" "*.Mask") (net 4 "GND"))
  (pad "13" thru_hole oval (at 0 15.24) (size 1.7 1.7) (drill 1) (layers "*.Cu" "*.Mask") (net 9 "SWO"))
  (pad "14" thru_hole oval (at -2.54 15.24) (size 1.7 1.7) (drill 1) (layers "*.Cu" "*.Mask") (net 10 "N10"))
  (pad "15" thru_hole oval (at 0 17.78) (size 1.7 1.7) (drill 1) (layers "*.Cu" "*.Mask") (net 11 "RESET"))
  (pad "16" thru_hole oval (at -2.54 17.78) (size 1.7 1.7) (drill 1) (layers "*.Cu" "*.Mask") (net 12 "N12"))
  (pad "17" thru_hole oval (at 0 20.32) (size 1.7 1.7) (drill 1) (layers "*.Cu" "*.Mask") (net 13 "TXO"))
  (pad "18" thru_hole oval (at -2.54 20.32) (size 1.7 1.7) (drill 1) (layers "*.Cu" "*.Mask") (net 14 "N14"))
  (pad "19" thru_hole oval (at 0 22.86) (size 1.7 1.7) (drill 1) (layers "*.Cu" "*.Mask") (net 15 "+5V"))
  (pad "20" thru_hole oval (at -2.54 22.86) (size 1.7 1.7) (drill 1) (layers "*.Cu" "*.Mask") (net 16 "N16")))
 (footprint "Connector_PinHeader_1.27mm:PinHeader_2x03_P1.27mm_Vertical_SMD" (layer "F.Cu") (at 132 105.44)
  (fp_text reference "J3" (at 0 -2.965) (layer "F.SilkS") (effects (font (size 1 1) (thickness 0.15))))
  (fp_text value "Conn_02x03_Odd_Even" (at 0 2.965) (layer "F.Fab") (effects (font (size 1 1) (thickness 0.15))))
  (fp_line (start -3.09 -1.9) (end -1.765 -1.9) (stroke (width 0.12) (type solid)) (layer "F.SilkS"))
  (fp_line (start -1.765 -1.965) (end -1.765 -1.9) (stroke (width 0.12) (type solid)) (layer "F.SilkS"))
  (fp_line (start -1.765 -1.965) (end 1.765 -1.965) (stroke (width 0.12) (type solid)) (layer "F.SilkS"))
  (fp_line (start -1.765 1.9) (end -1.765 1.965) (stroke (width 0.12) (type solid)) (layer "F.SilkS"))
  (fp_line (start -1.765 1.965) (end 1.765 1.965) (stroke (width 0.12) (type solid)) (layer "F.SilkS"))
  (fp_line (start 1.765 -1.965) (end 1.765 -1.9) (stroke (width 0.12) (type solid)) (layer "F.SilkS"))
  (fp_line (start 1.765 1.9) (end 1.765 1.965) (stroke (width 0.12) (type solid)) (layer "F.SilkS"))
  (pad "1" smd rect (at -1.95 -1.27) (size 2.4 0.74) (layers "F.Cu" "F.Paste" "F.Mask") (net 1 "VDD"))
  (pad "2" smd rect (at 1.95 -1.27) (size 2.4 0.74) (layers "F.Cu" "F.Paste" "F.Mask") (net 6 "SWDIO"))
  (pad "3" smd rect (at -1.95 0) (size 2.4 0.74) (layers "F.Cu" "F.Paste" "F.Mask") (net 11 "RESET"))
  (pad "4" smd rect (at 1.95 0) (size 2.4 0.74) (layers "F.Cu" "F.Paste" "F.Mask") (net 7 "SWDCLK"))
  (pad "5" smd rect (at -1.95 1.27) (size 2.4 0.74) (layers "F.Cu" "F.Paste" "F.Mask") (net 13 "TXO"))
  (pad "6" smd rect (at 1.95 1.27) (size 2.4 0.74) (layers "F.Cu" "F.Paste" "F.Mask") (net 4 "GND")))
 (gr_line (start 137 120) (end 137 93) (stroke (width 0.1) (type default)) (layer "Edge.Cuts"))
 (gr_line (start 137 93) (end 112 93) (stroke (width 0.1) (type default)) (layer "Edge.Cuts"))
 (gr_line (start 112 120) (end 137 120) (stroke (width 0.1) (type default)) (layer "Edge.Cuts"))
 (gr_line (start 112 93) (end 112 120) (stroke (width 0.1) (type default)) (layer "Edge.Cuts"))
 (segment (start 116.06 95.05) (end 117.31 96.3) (width 0.25) (layer "F.Cu") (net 1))
 (segment (start 129.04 104.19) (end 130.05 104.19) (width 0.25) (layer "F.Cu") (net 1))
 (segment (start 121.15 96.3) (end 129.04 104.19) (width 0.25) (layer "F.Cu") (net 1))
 (segment (start 117.31 96.3) (end 121.15 96.3) (width 0.25) (layer "F.Cu") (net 1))
 (segment (start 126 99.5) (end 131.9 99.5) (width 0.25) (layer "F.Cu") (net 6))
 (segment (start 116.06 102.67) (end 123.03 102.67) (width 0.25) (layer "F.Cu") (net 6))
 (segment (start 123.03 102.67) (end 124.4 101.3) (width 0.25) (layer "F.Cu") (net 6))
 (segment (start 131.9 99.5) (end 133.95 101.55) (width 0.25) (layer "F.Cu") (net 6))
 (segment (start 133.95 101.55) (end 133.95 104.17) (width 0.25) (layer "F.Cu") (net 6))
 (via (at 124.4 101.3) (size 0.8) (drill 0.4) (layers "F.Cu" "B.Cu") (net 6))
 (via (at 126 99.5) (size 0.8) (drill 0.4) (layers "F.Cu" "B.Cu") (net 6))
 (segment (start 126 99.7) (end 126 99.5) (width 0.25) (layer "B.Cu") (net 6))
 (segment (start 124.4 101.3) (end 126 99.7) (width 0.25) (layer "B.Cu") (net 6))
 (segment (start 133.95 106.71) (end 135.49 106.71) (width 0.25) (layer "F.Cu") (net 4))
 (segment (start 135.49 106.71) (end 135.5 106.7) (width 0.25) (layer "F.Cu") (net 4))
 (via (at 135.5 106.7) (size 0.8) (drill 0.4) (layers "F.Cu" "B.Cu") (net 4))
 (segment (start 133.95 105.46) (end 132.44 105.46) (width 0.25) (layer "F.Cu") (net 7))
 (segment (start 132.44 105.46) (end 131.95 105.95) (width 0.25) (layer "F.Cu") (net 7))
 (segment (start 131.95 105.95) (end 131.95 109.95) (width 0.25) (layer "F.Cu") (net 7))
 (segment (start 116.06 105.21) (end 117.35 106.5) (width 0.25) (layer "F.Cu") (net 7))
 (segment (start 131.95 109.95) (end 131.25 110.65) (width 0.25) (layer "F.Cu") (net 7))
 (segment (start 117.35 106.5) (end 120.5 106.5) (width 0.25) (layer "F.Cu") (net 7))
 (segment (start 131.25 110.65) (end 124.65 110.65) (width 0.25) (layer "F.Cu") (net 7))
 (via (at 120.5 106.5) (size 0.8) (drill 0.4) (layers "F.Cu" "B.Cu") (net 7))
 (via (at 124.65 110.65) (size 0.8) (drill 0.4) (layers "F.Cu" "B.Cu") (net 7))
 (segment (start 124.65 110.65) (end 120.5 106.5) (width 0.25) (layer "B.Cu") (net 7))
 (segment (start 124.72 106.71) (end 130.05 106.71) (width 0.25) (layer "F.Cu") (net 13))
 (segment (start 116.06 115.37) (end 124.72 106.71) (width 0.25) (layer "F.Cu") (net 13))
 (segment (start 123.45 105.44) (end 130.05 105.44) (width 0.25) (layer "F.Cu") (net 11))
 (segment (start 116.06 112.83) (end 123.45 105.44) (width 0.25) (layer "F.Cu") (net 11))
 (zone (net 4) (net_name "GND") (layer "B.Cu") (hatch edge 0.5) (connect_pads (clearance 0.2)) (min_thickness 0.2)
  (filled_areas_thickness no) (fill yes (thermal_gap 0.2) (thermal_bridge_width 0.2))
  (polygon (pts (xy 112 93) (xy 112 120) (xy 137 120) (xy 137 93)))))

